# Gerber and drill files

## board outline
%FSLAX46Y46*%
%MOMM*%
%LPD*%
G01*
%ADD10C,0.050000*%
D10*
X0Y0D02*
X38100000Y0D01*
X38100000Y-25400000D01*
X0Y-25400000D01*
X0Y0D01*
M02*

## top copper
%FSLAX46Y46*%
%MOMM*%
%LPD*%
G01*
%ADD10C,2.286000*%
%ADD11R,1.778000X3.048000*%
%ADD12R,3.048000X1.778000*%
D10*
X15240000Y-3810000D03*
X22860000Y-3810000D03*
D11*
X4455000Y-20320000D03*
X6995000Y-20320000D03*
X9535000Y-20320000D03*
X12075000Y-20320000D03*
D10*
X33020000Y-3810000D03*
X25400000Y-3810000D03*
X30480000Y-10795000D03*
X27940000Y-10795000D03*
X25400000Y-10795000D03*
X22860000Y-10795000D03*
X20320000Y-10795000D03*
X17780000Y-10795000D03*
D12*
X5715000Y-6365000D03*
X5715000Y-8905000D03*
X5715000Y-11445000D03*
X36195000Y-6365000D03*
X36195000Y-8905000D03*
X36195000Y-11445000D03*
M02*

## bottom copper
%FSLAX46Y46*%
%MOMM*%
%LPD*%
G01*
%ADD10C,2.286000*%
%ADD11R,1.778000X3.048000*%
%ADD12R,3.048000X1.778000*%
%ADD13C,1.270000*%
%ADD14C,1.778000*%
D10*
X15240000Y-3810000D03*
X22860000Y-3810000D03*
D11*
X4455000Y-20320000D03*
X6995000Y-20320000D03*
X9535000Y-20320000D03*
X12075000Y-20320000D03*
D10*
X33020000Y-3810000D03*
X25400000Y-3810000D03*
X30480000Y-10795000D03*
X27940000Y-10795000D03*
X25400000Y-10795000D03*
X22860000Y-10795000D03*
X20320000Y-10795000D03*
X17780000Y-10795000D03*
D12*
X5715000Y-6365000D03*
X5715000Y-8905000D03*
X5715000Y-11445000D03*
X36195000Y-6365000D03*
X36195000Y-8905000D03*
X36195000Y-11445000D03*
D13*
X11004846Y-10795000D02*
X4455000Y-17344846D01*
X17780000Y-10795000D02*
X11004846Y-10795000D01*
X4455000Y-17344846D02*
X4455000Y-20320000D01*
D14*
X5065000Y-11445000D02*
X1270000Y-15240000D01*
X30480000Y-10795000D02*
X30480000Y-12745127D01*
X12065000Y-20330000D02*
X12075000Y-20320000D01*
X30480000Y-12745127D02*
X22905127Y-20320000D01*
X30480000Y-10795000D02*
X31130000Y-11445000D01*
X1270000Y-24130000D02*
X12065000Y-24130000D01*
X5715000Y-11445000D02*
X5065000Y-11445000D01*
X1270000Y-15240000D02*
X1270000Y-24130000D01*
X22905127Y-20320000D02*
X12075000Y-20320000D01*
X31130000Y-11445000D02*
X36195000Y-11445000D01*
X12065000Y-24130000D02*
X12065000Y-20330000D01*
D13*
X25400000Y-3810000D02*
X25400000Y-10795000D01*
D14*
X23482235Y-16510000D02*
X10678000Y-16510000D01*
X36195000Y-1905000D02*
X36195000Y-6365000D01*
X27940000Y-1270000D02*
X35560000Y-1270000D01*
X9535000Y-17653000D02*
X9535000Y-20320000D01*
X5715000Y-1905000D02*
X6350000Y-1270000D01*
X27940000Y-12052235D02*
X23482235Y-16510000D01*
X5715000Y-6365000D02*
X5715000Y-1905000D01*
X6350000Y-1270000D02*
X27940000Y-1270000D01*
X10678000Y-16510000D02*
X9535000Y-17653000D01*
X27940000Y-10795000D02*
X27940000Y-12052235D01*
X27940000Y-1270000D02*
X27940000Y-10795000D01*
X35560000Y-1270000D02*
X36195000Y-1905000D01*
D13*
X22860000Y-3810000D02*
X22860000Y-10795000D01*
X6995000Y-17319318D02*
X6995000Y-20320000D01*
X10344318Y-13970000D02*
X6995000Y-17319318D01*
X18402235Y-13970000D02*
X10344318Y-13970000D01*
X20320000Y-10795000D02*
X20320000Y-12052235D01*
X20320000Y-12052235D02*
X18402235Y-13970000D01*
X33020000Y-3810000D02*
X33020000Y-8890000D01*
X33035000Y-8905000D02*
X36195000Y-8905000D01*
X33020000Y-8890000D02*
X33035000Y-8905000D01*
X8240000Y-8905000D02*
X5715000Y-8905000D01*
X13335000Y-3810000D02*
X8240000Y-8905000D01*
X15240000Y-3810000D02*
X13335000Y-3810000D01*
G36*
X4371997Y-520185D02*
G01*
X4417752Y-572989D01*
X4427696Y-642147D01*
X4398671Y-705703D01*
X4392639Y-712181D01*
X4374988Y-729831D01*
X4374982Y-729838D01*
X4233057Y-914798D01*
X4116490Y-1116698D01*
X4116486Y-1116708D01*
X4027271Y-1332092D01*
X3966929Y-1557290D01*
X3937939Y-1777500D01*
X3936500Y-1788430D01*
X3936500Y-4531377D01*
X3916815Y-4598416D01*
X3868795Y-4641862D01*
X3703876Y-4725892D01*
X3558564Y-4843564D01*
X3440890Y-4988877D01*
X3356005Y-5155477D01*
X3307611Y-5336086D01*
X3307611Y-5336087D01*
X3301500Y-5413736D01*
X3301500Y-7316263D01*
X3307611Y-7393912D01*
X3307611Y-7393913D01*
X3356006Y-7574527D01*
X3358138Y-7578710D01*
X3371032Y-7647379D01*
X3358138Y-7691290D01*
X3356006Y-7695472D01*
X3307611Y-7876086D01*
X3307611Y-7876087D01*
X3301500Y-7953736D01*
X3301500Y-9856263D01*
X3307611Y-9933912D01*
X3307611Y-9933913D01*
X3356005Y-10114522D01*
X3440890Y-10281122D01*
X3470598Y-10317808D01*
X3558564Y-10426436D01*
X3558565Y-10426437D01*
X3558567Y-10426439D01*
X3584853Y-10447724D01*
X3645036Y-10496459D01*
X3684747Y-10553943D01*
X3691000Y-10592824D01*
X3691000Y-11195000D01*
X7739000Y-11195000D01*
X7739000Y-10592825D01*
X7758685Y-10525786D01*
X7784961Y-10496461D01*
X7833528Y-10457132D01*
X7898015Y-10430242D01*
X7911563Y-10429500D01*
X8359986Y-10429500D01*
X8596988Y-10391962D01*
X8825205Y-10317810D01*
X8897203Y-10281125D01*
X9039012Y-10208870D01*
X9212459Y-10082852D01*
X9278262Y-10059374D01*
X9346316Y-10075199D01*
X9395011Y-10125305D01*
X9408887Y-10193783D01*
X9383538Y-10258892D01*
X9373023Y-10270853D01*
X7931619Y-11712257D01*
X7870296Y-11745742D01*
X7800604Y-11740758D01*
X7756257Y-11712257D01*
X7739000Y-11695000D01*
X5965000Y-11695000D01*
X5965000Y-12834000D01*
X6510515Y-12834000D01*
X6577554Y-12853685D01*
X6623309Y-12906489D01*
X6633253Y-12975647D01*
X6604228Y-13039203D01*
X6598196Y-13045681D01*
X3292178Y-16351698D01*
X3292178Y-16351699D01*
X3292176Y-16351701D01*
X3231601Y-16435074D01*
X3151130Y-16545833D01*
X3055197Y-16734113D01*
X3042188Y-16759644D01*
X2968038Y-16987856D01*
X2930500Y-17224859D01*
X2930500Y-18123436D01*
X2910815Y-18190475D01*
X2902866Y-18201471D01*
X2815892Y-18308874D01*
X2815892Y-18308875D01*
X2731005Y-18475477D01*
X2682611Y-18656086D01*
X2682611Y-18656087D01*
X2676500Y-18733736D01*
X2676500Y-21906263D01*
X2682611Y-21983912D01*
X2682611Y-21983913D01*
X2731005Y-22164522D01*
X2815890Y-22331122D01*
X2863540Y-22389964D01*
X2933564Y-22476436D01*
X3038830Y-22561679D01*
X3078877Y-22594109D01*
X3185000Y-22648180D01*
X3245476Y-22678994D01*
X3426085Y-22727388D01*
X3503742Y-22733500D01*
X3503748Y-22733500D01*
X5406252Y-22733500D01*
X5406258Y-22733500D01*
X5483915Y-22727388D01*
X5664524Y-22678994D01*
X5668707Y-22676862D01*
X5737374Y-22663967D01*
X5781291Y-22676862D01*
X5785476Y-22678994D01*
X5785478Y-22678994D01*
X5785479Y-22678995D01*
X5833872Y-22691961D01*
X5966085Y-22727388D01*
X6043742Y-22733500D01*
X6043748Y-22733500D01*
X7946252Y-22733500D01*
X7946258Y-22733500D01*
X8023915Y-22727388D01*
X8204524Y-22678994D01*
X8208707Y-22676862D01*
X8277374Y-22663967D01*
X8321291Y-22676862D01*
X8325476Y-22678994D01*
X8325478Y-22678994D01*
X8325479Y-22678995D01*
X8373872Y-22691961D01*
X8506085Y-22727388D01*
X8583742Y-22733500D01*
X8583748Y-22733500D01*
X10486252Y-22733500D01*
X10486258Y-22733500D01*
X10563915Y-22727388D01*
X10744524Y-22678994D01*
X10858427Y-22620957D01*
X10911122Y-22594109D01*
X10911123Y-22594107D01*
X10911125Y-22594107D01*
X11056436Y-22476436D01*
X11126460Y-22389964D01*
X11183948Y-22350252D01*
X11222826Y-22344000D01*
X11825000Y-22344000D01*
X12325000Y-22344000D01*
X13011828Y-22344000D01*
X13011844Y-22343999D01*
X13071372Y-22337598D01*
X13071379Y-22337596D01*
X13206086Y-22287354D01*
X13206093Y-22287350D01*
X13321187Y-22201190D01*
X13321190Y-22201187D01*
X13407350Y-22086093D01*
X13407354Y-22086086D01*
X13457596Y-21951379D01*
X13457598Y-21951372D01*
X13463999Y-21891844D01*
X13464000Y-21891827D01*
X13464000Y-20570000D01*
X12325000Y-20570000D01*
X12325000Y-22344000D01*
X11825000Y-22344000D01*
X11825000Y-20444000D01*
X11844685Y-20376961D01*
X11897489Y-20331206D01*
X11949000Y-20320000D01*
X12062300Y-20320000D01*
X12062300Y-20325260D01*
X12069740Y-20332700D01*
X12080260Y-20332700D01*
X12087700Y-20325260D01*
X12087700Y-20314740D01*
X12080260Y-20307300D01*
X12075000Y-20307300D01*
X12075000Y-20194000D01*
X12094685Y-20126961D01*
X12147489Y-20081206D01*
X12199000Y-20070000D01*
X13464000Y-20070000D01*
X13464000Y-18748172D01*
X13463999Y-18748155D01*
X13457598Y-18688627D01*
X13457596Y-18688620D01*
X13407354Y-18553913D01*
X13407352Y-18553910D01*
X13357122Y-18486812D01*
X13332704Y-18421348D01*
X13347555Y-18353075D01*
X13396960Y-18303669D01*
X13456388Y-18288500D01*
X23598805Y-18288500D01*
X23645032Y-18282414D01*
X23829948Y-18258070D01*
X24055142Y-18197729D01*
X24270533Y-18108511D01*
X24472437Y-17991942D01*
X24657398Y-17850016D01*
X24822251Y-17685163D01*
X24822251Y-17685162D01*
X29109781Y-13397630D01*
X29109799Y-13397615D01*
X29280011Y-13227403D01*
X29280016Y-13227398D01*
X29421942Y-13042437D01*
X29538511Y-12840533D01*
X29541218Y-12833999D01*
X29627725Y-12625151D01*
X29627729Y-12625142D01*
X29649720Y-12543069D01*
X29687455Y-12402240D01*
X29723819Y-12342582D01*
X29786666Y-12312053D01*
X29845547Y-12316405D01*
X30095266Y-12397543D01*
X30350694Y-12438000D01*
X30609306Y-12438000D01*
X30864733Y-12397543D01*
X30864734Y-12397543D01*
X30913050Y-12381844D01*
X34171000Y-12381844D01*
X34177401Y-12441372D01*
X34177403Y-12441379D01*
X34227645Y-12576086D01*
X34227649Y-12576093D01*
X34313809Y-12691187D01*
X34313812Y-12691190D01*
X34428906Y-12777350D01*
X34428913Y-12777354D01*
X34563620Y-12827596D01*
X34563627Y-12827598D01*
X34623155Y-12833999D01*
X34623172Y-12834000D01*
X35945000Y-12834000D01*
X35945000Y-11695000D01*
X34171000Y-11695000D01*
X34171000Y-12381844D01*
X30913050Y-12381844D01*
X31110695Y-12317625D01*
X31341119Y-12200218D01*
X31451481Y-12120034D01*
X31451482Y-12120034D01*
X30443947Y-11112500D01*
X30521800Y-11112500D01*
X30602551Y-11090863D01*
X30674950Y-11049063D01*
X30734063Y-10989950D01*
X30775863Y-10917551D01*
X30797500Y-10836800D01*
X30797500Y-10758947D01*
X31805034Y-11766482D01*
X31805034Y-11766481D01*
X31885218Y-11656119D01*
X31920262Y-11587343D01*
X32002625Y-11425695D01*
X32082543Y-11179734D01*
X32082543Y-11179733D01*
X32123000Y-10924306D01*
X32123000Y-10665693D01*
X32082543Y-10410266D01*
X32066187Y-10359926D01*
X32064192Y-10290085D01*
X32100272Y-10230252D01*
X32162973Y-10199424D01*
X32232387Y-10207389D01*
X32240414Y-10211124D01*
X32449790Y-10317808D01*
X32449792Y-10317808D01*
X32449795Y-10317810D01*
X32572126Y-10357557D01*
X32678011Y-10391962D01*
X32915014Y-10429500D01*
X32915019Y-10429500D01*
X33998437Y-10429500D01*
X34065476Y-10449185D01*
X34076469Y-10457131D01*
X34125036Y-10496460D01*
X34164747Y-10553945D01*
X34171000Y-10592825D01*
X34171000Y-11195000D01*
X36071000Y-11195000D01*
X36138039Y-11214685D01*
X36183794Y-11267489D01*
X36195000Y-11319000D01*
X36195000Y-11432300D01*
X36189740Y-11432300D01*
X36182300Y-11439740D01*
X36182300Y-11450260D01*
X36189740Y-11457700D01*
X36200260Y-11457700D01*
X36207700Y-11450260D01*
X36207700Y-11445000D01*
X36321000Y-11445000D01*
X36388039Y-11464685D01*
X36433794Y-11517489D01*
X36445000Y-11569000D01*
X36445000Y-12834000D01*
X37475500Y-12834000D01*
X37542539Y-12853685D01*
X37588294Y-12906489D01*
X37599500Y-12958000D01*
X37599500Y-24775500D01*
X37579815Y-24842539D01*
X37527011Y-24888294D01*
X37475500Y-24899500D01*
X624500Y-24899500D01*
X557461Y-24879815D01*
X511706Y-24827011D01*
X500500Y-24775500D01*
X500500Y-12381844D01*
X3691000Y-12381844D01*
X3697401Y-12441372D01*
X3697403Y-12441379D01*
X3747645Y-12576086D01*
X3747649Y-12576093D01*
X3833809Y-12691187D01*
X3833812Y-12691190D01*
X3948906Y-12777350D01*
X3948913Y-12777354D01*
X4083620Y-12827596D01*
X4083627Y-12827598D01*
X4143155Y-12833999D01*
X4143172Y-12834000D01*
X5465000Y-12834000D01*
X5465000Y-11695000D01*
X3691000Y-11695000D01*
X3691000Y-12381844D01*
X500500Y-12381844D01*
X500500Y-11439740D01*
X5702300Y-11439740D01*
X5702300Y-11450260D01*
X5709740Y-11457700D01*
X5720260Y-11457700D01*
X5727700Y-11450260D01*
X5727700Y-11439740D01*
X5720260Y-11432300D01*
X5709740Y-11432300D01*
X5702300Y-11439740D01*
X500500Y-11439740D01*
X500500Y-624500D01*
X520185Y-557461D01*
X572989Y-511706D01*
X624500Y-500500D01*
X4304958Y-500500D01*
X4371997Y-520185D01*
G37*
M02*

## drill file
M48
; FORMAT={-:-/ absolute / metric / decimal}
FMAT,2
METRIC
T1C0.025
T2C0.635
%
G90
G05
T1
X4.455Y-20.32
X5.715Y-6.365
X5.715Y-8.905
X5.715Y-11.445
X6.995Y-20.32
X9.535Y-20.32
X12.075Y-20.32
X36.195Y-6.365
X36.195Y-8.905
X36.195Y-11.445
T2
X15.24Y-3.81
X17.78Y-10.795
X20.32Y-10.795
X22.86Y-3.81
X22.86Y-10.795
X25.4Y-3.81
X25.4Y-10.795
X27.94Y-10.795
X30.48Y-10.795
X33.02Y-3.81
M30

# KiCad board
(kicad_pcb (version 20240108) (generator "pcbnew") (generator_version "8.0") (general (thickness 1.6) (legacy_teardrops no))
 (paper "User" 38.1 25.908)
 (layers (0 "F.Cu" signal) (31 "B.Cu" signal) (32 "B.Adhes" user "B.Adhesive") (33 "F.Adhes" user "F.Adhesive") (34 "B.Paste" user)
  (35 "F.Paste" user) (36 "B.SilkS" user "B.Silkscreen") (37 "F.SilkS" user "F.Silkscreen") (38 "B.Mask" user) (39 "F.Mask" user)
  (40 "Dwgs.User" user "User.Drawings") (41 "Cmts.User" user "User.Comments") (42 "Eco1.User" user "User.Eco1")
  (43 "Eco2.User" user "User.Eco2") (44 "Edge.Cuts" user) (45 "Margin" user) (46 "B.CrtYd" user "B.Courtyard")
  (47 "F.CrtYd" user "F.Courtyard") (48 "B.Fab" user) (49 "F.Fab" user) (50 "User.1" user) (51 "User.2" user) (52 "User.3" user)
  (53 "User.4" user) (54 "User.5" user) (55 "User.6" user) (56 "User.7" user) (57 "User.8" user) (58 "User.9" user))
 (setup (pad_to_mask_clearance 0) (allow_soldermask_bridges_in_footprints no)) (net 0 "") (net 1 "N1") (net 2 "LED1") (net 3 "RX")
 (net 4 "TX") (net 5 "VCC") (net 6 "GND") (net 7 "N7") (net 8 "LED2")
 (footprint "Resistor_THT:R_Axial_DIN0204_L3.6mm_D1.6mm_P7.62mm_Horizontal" (layer "F.Cu") (at 15.24 3.81)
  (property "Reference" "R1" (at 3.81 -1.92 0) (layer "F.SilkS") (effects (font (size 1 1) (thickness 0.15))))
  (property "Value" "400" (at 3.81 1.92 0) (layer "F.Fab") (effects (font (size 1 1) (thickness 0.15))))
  (pad "1" thru_hole circle (at 0 0) (size 2.286 2.286) (drill 0.635) (layers "*.Cu" "*.Mask") (remove_unused_layers no) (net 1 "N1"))
  (pad "2" thru_hole circle (at 7.62 0) (size 2.286 2.286) (drill 0.635) (layers "*.Cu" "*.Mask") (remove_unused_layers no) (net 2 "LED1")))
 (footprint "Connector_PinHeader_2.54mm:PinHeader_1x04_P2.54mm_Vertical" (layer "F.Cu") (at 4.455 20.32 90)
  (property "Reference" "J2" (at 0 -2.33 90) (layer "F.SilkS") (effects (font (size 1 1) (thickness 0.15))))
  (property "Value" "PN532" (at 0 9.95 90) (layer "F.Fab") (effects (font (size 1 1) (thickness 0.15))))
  (pad "1" thru_hole rect (at 0 0 90) (size 3.048 1.778) (drill 0.0254) (layers "*.Cu" "*.Mask") (remove_unused_layers no) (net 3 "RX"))
  (pad "2" thru_hole rect (at 0 2.54 90) (size 3.048 1.778) (drill 0.0254) (layers "*.Cu" "*.Mask") (remove_unused_layers no) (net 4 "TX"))
  (pad "3" thru_hole rect (at 0 5.08 90) (size 3.048 1.778) (drill 0.0254) (layers "*.Cu" "*.Mask") (remove_unused_layers no) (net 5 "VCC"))
  (pad "4" thru_hole rect (at 0 7.62 90) (size 3.048 1.778) (drill 0.0254) (layers "*.Cu" "*.Mask") (remove_unused_layers no) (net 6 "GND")))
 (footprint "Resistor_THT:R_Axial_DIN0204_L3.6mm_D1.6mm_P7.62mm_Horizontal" (layer "F.Cu") (at 33.02 3.81 180)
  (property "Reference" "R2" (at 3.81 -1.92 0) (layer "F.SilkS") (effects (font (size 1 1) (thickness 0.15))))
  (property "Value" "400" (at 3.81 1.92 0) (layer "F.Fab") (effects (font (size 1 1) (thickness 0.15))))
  (pad "1" thru_hole circle (at 0 0 180) (size 2.286 2.286) (drill 0.635) (layers "*.Cu" "*.Mask") (remove_unused_layers no) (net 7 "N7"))
  (pad "2" thru_hole circle (at 7.62 0 180) (size 2.286 2.286) (drill 0.635) (layers "*.Cu" "*.Mask") (remove_unused_layers no)
   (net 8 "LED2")))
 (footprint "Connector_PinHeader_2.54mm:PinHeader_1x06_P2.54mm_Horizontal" (layer "F.Cu") (at 30.48 10.795 -90)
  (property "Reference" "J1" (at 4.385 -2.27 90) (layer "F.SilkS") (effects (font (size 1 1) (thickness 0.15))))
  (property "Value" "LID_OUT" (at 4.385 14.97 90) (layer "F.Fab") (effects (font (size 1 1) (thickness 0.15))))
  (pad "1" thru_hole circle (at 0 0 270) (size 2.286 2.286) (drill 0.635) (layers "*.Cu" "*.Mask") (remove_unused_layers no) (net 6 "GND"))
  (pad "2" thru_hole circle (at 0 2.54 270) (size 2.286 2.286) (drill 0.635) (layers "*.Cu" "*.Mask") (remove_unused_layers no)
   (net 5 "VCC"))
  (pad "3" thru_hole circle (at 0 5.08 270) (size 2.286 2.286) (drill 0.635) (layers "*.Cu" "*.Mask") (remove_unused_layers no)
   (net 8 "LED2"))
  (pad "4" thru_hole circle (at 0 7.62 270) (size 2.286 2.286) (drill 0.635) (layers "*.Cu" "*.Mask") (remove_unused_layers no)
   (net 2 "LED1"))
  (pad "5" thru_hole circle (at 0 10.16 270) (size 2.286 2.286) (drill 0.635) (layers "*.Cu" "*.Mask") (remove_unused_layers no)
   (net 4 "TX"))
  (pad "6" thru_hole circle (at 0 12.7 270) (size 2.286 2.286) (drill 0.635) (layers "*.Cu" "*.Mask") (remove_unused_layers no) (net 3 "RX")))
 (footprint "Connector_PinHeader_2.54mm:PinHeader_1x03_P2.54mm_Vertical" (layer "F.Cu") (at 5.715 6.365)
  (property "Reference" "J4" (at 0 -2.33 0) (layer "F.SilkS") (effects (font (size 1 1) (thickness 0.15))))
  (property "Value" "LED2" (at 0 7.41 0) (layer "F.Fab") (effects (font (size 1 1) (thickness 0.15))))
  (pad "1" thru_hole rect (at 0 0) (size 3.048 1.778) (drill 0.0254) (layers "*.Cu" "*.Mask") (remove_unused_layers no) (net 5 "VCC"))
  (pad "2" thru_hole rect (at 0 2.54) (size 3.048 1.778) (drill 0.0254) (layers "*.Cu" "*.Mask") (remove_unused_layers no) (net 1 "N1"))
  (pad "3" thru_hole rect (at 0 5.08) (size 3.048 1.778) (drill 0.0254) (layers "*.Cu" "*.Mask") (remove_unused_layers no) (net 6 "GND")))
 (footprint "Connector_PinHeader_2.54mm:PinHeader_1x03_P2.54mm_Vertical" (layer "F.Cu") (at 36.195 6.365)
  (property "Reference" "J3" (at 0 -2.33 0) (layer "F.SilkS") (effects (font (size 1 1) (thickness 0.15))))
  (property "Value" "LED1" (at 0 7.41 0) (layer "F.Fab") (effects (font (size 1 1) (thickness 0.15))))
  (pad "1" thru_hole rect (at 0 0) (size 3.048 1.778) (drill 0.0254) (layers "*.Cu" "*.Mask") (remove_unused_layers no) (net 5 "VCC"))
  (pad "2" thru_hole rect (at 0 2.54) (size 3.048 1.778) (drill 0.0254) (layers "*.Cu" "*.Mask") (remove_unused_layers no) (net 7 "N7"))
  (pad "3" thru_hole rect (at 0 5.08) (size 3.048 1.778) (drill 0.0254) (layers "*.Cu" "*.Mask") (remove_unused_layers no) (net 6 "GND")))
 (gr_rect (start 0 0) (end 38.1 25.4) (stroke (width 0.05) (type default)) (fill none) (layer "Edge.Cuts"))
 (segment (start 11.004846 10.795) (end 4.455 17.344846) (width 1.27) (layer "B.Cu") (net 3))
 (segment (start 17.78 10.795) (end 11.004846 10.795) (width 1.27) (layer "B.Cu") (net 3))
 (segment (start 4.455 17.344846) (end 4.455 20.32) (width 1.27) (layer "B.Cu") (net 3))
 (segment (start 5.065 11.445) (end 1.27 15.24) (width 1.778) (layer "B.Cu") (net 6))
 (segment (start 30.48 10.795) (end 30.48 12.745127) (width 1.778) (layer "B.Cu") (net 6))
 (segment (start 12.065 20.33) (end 12.075 20.32) (width 1.778) (layer "B.Cu") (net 6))
 (segment (start 30.48 12.745127) (end 22.905127 20.32) (width 1.778) (layer "B.Cu") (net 6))
 (segment (start 30.48 10.795) (end 31.13 11.445) (width 1.778) (layer "B.Cu") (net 6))
 (segment (start 1.27 24.13) (end 12.065 24.13) (width 1.778) (layer "B.Cu") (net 6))
 (segment (start 5.715 11.445) (end 5.065 11.445) (width 1.778) (layer "B.Cu") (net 6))
 (segment (start 1.27 15.24) (end 1.27 24.13) (width 1.778) (layer "B.Cu") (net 6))
 (segment (start 22.905127 20.32) (end 12.075 20.32) (width 1.778) (layer "B.Cu") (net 6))
 (segment (start 31.13 11.445) (end 36.195 11.445) (width 1.778) (layer "B.Cu") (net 6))
 (segment (start 12.065 24.13) (end 12.065 20.33) (width 1.778) (layer "B.Cu") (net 6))
 (segment (start 25.4 3.81) (end 25.4 10.795) (width 1.27) (layer "B.Cu") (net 8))
 (segment (start 23.482235 16.51) (end 10.678 16.51) (width 1.778) (layer "B.Cu") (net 5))
 (segment (start 36.195 1.905) (end 36.195 6.365) (width 1.778) (layer "B.Cu") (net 5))
 (segment (start 27.94 1.27) (end 35.56 1.27) (width 1.778) (layer "B.Cu") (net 5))
 (segment (start 9.535 17.653) (end 9.535 20.32) (width 1.778) (layer "B.Cu") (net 5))
 (segment (start 5.715 1.905) (end 6.35 1.27) (width 1.778) (layer "B.Cu") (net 5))
 (segment (start 27.94 12.052235) (end 23.482235 16.51) (width 1.778) (layer "B.Cu") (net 5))
 (segment (start 5.715 6.365) (end 5.715 1.905) (width 1.778) (layer "B.Cu") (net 5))
 (segment (start 6.35 1.27) (end 27.94 1.27) (width 1.778) (layer "B.Cu") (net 5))
 (segment (start 10.678 16.51) (end 9.535 17.653) (width 1.778) (layer "B.Cu") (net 5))
 (segment (start 27.94 10.795) (end 27.94 12.052235) (width 1.778) (layer "B.Cu") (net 5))
 (segment (start 27.94 1.27) (end 27.94 10.795) (width 1.778) (layer "B.Cu") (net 5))
 (segment (start 35.56 1.27) (end 36.195 1.905) (width 1.778) (layer "B.Cu") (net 5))
 (segment (start 22.86 3.81) (end 22.86 10.795) (width 1.27) (layer "B.Cu") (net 2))
 (segment (start 6.995 17.319318) (end 6.995 20.32) (width 1.27) (layer "B.Cu") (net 4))
 (segment (start 10.344318 13.97) (end 6.995 17.319318) (width 1.27) (layer "B.Cu") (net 4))
 (segment (start 18.402235 13.97) (end 10.344318 13.97) (width 1.27) (layer "B.Cu") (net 4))
 (segment (start 20.32 10.795) (end 20.32 12.052235) (width 1.27) (layer "B.Cu") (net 4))
 (segment (start 20.32 12.052235) (end 18.402235 13.97) (width 1.27) (layer "B.Cu") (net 4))
 (segment (start 33.02 3.81) (end 33.02 8.89) (width 1.27) (layer "B.Cu") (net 7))
 (segment (start 33.035 8.905) (end 36.195 8.905) (width 1.27) (layer "B.Cu") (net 7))
 (segment (start 33.02 8.89) (end 33.035 8.905) (width 1.27) (layer "B.Cu") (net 7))
 (segment (start 8.24 8.905) (end 5.715 8.905) (width 1.27) (layer "B.Cu") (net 1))
 (segment (start 13.335 3.81) (end 8.24 8.905) (width 1.27) (layer "B.Cu") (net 1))
 (segment (start 15.24 3.81) (end 13.335 3.81) (width 1.27) (layer "B.Cu") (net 1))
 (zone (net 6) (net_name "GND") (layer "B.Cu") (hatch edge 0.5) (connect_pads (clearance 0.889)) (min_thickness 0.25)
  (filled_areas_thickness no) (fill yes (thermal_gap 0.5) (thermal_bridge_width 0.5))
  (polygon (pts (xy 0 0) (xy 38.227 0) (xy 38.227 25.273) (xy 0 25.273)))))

